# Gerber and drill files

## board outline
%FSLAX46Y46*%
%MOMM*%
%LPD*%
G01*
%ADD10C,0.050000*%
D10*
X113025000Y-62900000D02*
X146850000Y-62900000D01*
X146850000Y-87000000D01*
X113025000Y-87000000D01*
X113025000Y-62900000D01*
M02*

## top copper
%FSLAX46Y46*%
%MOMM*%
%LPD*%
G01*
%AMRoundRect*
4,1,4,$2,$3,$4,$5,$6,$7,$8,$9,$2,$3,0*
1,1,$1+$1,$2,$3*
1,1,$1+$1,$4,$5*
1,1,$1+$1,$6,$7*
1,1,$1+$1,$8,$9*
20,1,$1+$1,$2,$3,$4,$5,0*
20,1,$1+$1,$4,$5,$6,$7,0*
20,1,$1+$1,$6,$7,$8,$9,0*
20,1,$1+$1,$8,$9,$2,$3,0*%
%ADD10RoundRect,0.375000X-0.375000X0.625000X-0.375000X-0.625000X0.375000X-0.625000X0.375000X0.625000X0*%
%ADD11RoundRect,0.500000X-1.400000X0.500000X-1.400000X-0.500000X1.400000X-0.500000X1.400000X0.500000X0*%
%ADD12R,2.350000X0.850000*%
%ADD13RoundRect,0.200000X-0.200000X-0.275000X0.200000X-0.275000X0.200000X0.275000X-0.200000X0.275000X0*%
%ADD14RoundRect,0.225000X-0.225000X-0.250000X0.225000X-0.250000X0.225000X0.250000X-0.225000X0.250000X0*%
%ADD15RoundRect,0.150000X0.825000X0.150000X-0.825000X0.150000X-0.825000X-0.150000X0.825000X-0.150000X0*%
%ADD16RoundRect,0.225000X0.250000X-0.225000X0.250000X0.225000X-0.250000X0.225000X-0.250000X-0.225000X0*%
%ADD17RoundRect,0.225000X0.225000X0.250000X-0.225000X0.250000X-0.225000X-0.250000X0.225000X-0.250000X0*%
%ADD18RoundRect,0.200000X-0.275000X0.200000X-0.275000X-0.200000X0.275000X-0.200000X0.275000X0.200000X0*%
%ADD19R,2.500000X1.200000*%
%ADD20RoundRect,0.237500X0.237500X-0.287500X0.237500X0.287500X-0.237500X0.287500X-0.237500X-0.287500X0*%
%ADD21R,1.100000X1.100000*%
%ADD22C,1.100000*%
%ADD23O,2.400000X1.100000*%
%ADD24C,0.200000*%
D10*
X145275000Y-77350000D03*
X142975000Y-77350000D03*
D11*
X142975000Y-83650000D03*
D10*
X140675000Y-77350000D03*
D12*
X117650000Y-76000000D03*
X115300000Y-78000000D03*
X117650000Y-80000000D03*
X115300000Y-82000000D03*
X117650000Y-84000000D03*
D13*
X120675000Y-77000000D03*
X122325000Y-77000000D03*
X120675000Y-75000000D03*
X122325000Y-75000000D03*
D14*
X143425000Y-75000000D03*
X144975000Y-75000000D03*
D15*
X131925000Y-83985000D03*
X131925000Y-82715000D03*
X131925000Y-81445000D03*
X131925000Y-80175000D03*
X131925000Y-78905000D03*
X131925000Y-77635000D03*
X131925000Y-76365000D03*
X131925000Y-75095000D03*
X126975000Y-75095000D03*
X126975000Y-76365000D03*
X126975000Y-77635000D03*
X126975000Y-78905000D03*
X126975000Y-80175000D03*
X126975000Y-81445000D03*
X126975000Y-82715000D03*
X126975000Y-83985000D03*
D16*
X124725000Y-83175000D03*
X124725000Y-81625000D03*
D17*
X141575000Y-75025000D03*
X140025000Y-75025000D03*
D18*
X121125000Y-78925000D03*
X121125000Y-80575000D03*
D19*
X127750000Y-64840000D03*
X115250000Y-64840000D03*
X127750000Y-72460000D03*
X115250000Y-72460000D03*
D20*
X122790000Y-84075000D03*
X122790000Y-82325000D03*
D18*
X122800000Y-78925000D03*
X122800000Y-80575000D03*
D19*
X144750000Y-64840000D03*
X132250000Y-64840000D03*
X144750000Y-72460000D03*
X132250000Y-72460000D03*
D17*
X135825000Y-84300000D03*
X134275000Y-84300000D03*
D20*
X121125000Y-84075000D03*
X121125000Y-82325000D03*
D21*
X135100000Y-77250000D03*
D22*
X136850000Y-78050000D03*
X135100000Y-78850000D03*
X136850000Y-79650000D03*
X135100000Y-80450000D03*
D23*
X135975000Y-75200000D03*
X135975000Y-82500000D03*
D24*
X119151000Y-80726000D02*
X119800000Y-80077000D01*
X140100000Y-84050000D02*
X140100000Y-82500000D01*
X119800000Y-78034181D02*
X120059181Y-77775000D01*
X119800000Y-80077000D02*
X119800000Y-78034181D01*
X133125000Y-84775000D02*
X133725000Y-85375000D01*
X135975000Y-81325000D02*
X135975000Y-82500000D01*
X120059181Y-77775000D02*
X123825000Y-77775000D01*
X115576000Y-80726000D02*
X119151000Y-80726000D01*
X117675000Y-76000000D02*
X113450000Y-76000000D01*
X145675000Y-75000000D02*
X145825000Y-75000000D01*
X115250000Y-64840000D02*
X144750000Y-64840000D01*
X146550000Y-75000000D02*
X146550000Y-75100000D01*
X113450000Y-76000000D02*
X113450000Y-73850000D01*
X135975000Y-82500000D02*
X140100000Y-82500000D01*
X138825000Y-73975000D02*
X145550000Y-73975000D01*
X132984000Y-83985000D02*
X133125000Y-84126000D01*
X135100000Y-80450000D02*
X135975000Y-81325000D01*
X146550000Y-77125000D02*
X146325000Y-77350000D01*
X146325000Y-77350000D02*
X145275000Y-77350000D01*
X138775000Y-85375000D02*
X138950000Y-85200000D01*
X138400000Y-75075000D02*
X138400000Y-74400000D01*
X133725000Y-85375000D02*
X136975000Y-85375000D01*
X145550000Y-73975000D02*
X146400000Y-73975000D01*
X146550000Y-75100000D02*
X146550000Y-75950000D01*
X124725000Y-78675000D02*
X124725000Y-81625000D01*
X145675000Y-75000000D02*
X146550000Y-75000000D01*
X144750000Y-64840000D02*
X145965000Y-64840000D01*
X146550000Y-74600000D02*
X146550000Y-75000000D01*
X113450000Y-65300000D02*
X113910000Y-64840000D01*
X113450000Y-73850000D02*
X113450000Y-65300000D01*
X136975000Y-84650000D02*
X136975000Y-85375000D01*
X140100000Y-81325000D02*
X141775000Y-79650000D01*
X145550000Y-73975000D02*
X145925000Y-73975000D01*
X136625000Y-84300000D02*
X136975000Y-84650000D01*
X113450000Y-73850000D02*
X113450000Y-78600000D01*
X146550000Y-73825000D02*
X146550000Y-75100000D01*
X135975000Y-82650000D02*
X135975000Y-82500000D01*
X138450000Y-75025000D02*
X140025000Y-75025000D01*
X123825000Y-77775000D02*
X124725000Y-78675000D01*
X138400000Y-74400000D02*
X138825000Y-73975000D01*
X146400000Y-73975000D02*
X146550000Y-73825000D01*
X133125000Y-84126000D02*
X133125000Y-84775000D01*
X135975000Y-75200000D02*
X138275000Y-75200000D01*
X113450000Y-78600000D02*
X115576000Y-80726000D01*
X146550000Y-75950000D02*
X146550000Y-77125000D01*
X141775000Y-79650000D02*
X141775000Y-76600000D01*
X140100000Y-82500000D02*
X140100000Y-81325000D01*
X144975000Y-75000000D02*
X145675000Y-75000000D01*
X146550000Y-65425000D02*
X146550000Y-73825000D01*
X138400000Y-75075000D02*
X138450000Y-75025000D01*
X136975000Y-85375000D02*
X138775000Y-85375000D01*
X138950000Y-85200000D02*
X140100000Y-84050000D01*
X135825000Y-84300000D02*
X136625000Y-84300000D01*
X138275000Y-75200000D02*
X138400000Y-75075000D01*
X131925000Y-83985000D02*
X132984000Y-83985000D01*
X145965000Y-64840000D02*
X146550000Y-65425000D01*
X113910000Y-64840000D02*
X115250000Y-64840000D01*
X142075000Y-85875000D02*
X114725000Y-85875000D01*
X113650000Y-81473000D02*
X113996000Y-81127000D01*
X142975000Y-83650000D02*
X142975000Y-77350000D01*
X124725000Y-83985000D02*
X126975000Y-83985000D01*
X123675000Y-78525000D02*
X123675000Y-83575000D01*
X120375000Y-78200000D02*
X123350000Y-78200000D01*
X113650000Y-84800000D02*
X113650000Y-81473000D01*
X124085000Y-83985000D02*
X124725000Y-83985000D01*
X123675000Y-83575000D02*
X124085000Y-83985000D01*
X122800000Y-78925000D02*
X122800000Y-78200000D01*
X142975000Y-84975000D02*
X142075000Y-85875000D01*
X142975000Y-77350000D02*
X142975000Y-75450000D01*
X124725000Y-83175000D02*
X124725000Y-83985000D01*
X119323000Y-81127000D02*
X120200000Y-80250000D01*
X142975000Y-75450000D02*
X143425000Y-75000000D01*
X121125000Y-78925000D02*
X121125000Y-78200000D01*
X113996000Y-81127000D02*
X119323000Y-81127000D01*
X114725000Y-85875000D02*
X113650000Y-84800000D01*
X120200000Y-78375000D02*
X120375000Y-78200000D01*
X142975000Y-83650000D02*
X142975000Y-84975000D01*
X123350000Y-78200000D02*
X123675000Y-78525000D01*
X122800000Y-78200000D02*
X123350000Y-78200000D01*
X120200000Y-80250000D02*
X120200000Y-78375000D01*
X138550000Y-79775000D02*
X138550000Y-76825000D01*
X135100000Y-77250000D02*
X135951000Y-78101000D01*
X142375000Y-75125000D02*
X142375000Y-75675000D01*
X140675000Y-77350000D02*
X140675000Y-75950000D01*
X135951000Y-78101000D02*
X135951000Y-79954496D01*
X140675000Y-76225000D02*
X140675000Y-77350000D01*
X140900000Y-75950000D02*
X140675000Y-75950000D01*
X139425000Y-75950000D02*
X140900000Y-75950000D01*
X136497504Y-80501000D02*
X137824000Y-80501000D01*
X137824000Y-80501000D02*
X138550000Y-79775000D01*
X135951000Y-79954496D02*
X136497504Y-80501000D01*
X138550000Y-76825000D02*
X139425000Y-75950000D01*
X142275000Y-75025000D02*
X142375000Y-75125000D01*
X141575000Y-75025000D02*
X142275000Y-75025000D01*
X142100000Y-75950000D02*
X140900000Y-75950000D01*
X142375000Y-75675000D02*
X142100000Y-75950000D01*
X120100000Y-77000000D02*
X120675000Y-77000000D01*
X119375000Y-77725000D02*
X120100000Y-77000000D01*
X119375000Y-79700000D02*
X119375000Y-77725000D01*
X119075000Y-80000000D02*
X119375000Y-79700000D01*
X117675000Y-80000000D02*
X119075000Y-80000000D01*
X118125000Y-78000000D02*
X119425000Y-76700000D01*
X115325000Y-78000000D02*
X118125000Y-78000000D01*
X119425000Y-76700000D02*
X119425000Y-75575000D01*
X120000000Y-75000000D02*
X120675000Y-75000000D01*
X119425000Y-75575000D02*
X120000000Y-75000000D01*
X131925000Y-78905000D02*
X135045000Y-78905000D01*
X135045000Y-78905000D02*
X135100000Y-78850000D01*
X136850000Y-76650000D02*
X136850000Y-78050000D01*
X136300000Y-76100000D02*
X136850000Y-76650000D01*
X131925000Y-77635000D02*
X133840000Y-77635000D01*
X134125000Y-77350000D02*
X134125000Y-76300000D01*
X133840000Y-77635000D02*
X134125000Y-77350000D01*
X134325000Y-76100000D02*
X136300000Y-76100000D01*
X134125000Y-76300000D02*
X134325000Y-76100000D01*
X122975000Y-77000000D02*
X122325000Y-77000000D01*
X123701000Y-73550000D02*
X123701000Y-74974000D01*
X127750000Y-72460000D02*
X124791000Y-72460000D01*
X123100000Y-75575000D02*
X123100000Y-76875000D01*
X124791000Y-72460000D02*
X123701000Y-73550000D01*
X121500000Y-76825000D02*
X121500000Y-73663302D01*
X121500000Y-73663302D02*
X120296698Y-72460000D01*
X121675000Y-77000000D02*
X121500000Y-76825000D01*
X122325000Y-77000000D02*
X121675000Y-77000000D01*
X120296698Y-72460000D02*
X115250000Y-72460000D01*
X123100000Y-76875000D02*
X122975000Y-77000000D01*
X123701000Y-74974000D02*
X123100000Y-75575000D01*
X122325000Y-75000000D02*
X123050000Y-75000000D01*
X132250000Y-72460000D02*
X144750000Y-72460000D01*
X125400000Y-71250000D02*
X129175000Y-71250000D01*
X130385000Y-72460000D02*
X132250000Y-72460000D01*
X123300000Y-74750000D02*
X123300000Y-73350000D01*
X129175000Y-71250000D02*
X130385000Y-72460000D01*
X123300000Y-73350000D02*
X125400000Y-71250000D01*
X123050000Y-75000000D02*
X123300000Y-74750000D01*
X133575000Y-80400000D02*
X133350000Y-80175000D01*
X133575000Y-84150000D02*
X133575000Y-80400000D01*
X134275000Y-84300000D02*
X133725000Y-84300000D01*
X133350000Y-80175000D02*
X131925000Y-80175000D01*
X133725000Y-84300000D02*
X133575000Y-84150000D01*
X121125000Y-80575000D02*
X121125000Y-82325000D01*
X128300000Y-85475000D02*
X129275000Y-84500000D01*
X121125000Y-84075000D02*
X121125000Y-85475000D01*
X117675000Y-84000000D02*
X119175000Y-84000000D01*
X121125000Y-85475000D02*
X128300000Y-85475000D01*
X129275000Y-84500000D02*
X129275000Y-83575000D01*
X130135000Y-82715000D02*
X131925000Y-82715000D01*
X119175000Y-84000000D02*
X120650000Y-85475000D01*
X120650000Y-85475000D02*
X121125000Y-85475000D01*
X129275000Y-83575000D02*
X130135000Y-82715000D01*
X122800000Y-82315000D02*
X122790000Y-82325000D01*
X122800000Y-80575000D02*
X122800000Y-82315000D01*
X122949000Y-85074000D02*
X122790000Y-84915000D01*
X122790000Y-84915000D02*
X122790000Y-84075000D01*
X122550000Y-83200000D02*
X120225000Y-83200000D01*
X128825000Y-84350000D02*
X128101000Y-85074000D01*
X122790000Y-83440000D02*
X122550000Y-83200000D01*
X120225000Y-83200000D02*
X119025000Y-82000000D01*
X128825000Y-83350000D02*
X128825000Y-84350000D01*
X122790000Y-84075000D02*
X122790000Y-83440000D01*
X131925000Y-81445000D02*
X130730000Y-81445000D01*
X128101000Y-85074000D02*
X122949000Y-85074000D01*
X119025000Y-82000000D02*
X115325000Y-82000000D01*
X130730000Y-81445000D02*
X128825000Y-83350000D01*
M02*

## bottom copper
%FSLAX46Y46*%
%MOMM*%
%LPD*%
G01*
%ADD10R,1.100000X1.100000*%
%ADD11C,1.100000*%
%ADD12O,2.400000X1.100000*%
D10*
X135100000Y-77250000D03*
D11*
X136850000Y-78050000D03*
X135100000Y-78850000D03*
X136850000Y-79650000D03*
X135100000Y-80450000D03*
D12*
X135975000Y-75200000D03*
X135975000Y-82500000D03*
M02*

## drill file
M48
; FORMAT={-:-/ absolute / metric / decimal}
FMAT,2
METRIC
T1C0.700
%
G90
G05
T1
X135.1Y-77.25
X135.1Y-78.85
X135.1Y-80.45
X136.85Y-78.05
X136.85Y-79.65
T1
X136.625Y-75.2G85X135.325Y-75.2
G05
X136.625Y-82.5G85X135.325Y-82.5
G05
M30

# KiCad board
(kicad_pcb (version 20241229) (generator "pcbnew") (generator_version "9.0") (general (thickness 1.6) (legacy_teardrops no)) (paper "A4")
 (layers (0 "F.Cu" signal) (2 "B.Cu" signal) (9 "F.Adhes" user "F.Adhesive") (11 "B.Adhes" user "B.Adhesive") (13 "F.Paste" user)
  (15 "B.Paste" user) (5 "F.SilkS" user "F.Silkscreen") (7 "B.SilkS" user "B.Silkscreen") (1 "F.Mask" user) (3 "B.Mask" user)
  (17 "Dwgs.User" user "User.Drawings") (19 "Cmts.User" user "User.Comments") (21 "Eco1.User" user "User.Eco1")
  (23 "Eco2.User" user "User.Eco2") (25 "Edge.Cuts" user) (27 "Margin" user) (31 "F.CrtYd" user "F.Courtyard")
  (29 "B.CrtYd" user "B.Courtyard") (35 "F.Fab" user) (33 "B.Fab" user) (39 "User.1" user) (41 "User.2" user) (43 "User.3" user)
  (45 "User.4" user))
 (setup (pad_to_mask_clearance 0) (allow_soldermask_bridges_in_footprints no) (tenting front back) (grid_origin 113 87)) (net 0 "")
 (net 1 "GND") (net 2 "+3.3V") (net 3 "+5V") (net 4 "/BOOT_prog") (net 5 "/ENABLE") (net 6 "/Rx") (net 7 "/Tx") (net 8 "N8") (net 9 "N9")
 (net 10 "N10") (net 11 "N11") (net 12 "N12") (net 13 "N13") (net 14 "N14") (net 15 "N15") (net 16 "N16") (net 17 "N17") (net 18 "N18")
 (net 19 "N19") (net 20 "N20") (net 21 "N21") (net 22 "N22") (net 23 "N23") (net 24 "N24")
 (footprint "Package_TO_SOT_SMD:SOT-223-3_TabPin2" (layer "F.Cu") (at 142.975 80.5 -90)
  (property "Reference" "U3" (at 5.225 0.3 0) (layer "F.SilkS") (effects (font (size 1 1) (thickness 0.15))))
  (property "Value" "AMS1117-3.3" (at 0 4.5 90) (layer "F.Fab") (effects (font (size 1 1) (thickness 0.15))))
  (pad "1" smd roundrect (at -3.15 -2.3 270) (size 2 1.5) (layers "F.Cu" "F.Mask" "F.Paste") (roundrect_rratio 0.25) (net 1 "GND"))
  (pad "2" smd roundrect (at -3.15 0 270) (size 2 1.5) (layers "F.Cu" "F.Mask" "F.Paste") (roundrect_rratio 0.25) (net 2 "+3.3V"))
  (pad "2" smd roundrect (at 3.15 0 270) (size 2 3.8) (layers "F.Cu" "F.Mask" "F.Paste") (roundrect_rratio 0.25) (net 2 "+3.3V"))
  (pad "3" smd roundrect (at -3.15 2.3 270) (size 2 1.5) (layers "F.Cu" "F.Mask" "F.Paste") (roundrect_rratio 0.25) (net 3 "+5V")))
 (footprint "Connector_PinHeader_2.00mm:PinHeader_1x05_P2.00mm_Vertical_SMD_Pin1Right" (layer "F.Cu") (at 116.475 80)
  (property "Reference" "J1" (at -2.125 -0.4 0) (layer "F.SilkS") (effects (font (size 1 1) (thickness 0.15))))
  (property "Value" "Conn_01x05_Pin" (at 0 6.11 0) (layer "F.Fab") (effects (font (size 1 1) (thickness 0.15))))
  (pad "1" smd rect (at 1.175 -4) (size 2.35 0.85) (layers "F.Cu" "F.Mask" "F.Paste") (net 1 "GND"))
  (pad "2" smd rect (at -1.175 -2) (size 2.35 0.85) (layers "F.Cu" "F.Mask" "F.Paste") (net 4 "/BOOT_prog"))
  (pad "3" smd rect (at 1.175 0) (size 2.35 0.85) (layers "F.Cu" "F.Mask" "F.Paste") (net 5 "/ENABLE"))
  (pad "4" smd rect (at -1.175 2) (size 2.35 0.85) (layers "F.Cu" "F.Mask" "F.Paste") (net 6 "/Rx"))
  (pad "5" smd rect (at 1.175 4) (size 2.35 0.85) (layers "F.Cu" "F.Mask" "F.Paste") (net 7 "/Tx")))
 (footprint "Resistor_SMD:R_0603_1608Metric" (layer "F.Cu") (at 121.5 77)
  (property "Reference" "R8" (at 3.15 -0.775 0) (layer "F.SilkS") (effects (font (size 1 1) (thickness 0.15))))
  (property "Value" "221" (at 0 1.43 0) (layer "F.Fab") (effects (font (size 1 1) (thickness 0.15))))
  (pad "1" smd roundrect (at -0.825 0) (size 0.8 0.95) (layers "F.Cu" "F.Mask" "F.Paste") (roundrect_rratio 0.25) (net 5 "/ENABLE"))
  (pad "2" smd roundrect (at 0.825 0) (size 0.8 0.95) (layers "F.Cu" "F.Mask" "F.Paste") (roundrect_rratio 0.25) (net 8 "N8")))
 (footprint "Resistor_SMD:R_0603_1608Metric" (layer "F.Cu") (at 121.5 75)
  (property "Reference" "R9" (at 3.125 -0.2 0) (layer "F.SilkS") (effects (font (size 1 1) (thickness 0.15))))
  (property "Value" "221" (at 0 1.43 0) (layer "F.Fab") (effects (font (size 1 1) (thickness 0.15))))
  (pad "1" smd roundrect (at -0.825 0) (size 0.8 0.95) (layers "F.Cu" "F.Mask" "F.Paste") (roundrect_rratio 0.25) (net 4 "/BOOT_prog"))
  (pad "2" smd roundrect (at 0.825 0) (size 0.8 0.95) (layers "F.Cu" "F.Mask" "F.Paste") (roundrect_rratio 0.25) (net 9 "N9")))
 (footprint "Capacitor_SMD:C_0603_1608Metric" (layer "F.Cu") (at 144.2 75)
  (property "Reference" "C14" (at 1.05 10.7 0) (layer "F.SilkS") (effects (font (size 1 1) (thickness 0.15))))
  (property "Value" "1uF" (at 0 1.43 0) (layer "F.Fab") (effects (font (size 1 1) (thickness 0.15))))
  (pad "1" smd roundrect (at -0.775 0) (size 0.9 0.95) (layers "F.Cu" "F.Mask" "F.Paste") (roundrect_rratio 0.25) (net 2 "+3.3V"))
  (pad "2" smd roundrect (at 0.775 0) (size 0.9 0.95) (layers "F.Cu" "F.Mask" "F.Paste") (roundrect_rratio 0.25) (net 1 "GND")))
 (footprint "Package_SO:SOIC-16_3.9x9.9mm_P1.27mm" (layer "F.Cu") (at 129.45 79.54 180)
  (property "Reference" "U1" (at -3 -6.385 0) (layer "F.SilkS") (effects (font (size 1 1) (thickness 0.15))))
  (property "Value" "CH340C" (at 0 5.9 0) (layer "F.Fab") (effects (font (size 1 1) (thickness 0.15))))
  (pad "1" smd roundrect (at -2.475 -4.445 180) (size 1.95 0.6) (layers "F.Cu" "F.Mask" "F.Paste") (roundrect_rratio 0.25) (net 1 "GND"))
  (pad "2" smd roundrect (at -2.475 -3.175 180) (size 1.95 0.6) (layers "F.Cu" "F.Mask" "F.Paste") (roundrect_rratio 0.25) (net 7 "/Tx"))
  (pad "3" smd roundrect (at -2.475 -1.905 180) (size 1.95 0.6) (layers "F.Cu" "F.Mask" "F.Paste") (roundrect_rratio 0.25) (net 6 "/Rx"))
  (pad "4" smd roundrect (at -2.475 -0.635 180) (size 1.95 0.6) (layers "F.Cu" "F.Mask" "F.Paste") (roundrect_rratio 0.25) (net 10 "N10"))
  (pad "5" smd roundrect (at -2.475 0.635 180) (size 1.95 0.6) (layers "F.Cu" "F.Mask" "F.Paste") (roundrect_rratio 0.25) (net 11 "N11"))
  (pad "6" smd roundrect (at -2.475 1.905 180) (size 1.95 0.6) (layers "F.Cu" "F.Mask" "F.Paste") (roundrect_rratio 0.25) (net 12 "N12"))
  (pad "7" smd roundrect (at -2.475 3.175 180) (size 1.95 0.6) (layers "F.Cu" "F.Mask" "F.Paste") (roundrect_rratio 0.25) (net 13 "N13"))
  (pad "8" smd roundrect (at -2.475 4.445 180) (size 1.95 0.6) (layers "F.Cu" "F.Mask" "F.Paste") (roundrect_rratio 0.25) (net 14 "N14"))
  (pad "9" smd roundrect (at 2.475 4.445 180) (size 1.95 0.6) (layers "F.Cu" "F.Mask" "F.Paste") (roundrect_rratio 0.25) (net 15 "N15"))
  (pad "10" smd roundrect (at 2.475 3.175 180) (size 1.95 0.6) (layers "F.Cu" "F.Mask" "F.Paste") (roundrect_rratio 0.25) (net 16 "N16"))
  (pad "11" smd roundrect (at 2.475 1.905 180) (size 1.95 0.6) (layers "F.Cu" "F.Mask" "F.Paste") (roundrect_rratio 0.25) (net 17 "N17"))
  (pad "12" smd roundrect (at 2.475 0.635 180) (size 1.95 0.6) (layers "F.Cu" "F.Mask" "F.Paste") (roundrect_rratio 0.25) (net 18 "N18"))
  (pad "13" smd roundrect (at 2.475 -0.635 180) (size 1.95 0.6) (layers "F.Cu" "F.Mask" "F.Paste") (roundrect_rratio 0.25) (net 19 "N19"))
  (pad "14" smd roundrect (at 2.475 -1.905 180) (size 1.95 0.6) (layers "F.Cu" "F.Mask" "F.Paste") (roundrect_rratio 0.25) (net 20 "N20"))
  (pad "15" smd roundrect (at 2.475 -3.175 180) (size 1.95 0.6) (layers "F.Cu" "F.Mask" "F.Paste") (roundrect_rratio 0.25) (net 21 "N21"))
  (pad "16" smd roundrect (at 2.475 -4.445 180) (size 1.95 0.6) (layers "F.Cu" "F.Mask" "F.Paste") (roundrect_rratio 0.25) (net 2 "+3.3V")))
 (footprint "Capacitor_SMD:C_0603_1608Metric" (layer "F.Cu") (at 124.725 82.4 90)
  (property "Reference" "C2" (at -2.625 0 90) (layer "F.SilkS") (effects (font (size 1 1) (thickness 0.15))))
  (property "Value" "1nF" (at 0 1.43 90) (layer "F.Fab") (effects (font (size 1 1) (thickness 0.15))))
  (pad "1" smd roundrect (at -0.775 0 90) (size 0.9 0.95) (layers "F.Cu" "F.Mask" "F.Paste") (roundrect_rratio 0.25) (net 2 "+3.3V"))
  (pad "2" smd roundrect (at 0.775 0 90) (size 0.9 0.95) (layers "F.Cu" "F.Mask" "F.Paste") (roundrect_rratio 0.25) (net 1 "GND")))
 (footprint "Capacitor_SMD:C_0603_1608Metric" (layer "F.Cu") (at 140.8 75.025 180)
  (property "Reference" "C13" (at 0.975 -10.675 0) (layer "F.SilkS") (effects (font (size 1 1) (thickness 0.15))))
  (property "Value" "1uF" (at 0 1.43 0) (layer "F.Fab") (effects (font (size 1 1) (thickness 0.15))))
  (pad "1" smd roundrect (at -0.775 0 180) (size 0.9 0.95) (layers "F.Cu" "F.Mask" "F.Paste") (roundrect_rratio 0.25) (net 3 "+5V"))
  (pad "2" smd roundrect (at 0.775 0 180) (size 0.9 0.95) (layers "F.Cu" "F.Mask" "F.Paste") (roundrect_rratio 0.25) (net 1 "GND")))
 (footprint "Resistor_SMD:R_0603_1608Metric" (layer "F.Cu") (at 121.125 79.75 -90)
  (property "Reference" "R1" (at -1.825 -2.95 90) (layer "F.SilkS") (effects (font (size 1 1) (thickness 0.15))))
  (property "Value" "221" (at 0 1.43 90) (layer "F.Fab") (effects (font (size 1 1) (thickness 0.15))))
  (pad "1" smd roundrect (at -0.825 0 270) (size 0.8 0.95) (layers "F.Cu" "F.Mask" "F.Paste") (roundrect_rratio 0.25) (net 2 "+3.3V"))
  (pad "2" smd roundrect (at 0.825 0 270) (size 0.8 0.95) (layers "F.Cu" "F.Mask" "F.Paste") (roundrect_rratio 0.25) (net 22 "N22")))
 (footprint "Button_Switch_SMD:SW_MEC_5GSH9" (layer "F.Cu") (at 121.5 68.65 -90)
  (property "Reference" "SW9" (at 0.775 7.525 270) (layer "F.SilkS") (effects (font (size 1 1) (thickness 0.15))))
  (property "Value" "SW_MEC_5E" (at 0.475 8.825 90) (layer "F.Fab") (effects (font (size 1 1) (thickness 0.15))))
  (pad "1" smd rect (at -3.81 -6.25) (size 2.5 1.2) (layers "F.Cu" "F.Mask" "F.Paste") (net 1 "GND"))
  (pad "2" smd rect (at -3.81 6.25) (size 2.5 1.2) (layers "F.Cu" "F.Mask" "F.Paste") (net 1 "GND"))
  (pad "3" smd rect (at 3.81 -6.25) (size 2.5 1.2) (layers "F.Cu" "F.Mask" "F.Paste") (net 8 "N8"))
  (pad "4" smd rect (at 3.81 6.25) (size 2.5 1.2) (layers "F.Cu" "F.Mask" "F.Paste") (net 8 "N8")))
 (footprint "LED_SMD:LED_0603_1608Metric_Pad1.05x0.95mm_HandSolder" (layer "F.Cu") (at 122.79 83.2 90)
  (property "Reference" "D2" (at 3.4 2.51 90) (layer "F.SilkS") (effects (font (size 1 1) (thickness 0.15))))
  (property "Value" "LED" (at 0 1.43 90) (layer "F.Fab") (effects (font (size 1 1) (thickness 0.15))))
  (pad "1" smd roundrect (at -0.875 0 90) (size 1.05 0.95) (layers "F.Cu" "F.Mask" "F.Paste") (roundrect_rratio 0.25) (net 6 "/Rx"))
  (pad "2" smd roundrect (at 0.875 0 90) (size 1.05 0.95) (layers "F.Cu" "F.Mask" "F.Paste") (roundrect_rratio 0.25) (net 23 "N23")))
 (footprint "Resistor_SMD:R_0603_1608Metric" (layer "F.Cu") (at 122.8 79.75 -90)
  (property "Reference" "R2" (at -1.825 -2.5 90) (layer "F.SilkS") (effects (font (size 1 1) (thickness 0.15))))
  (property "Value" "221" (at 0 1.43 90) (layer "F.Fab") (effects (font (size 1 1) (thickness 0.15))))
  (pad "1" smd roundrect (at -0.825 0 270) (size 0.8 0.95) (layers "F.Cu" "F.Mask" "F.Paste") (roundrect_rratio 0.25) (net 2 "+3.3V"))
  (pad "2" smd roundrect (at 0.825 0 270) (size 0.8 0.95) (layers "F.Cu" "F.Mask" "F.Paste") (roundrect_rratio 0.25) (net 23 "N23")))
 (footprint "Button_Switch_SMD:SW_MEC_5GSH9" (layer "F.Cu") (at 138.5 68.65 -90)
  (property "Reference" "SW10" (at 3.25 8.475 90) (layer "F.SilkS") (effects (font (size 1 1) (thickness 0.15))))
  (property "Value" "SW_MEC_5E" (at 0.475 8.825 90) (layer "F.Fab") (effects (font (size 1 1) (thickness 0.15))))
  (pad "1" smd rect (at -3.81 -6.25) (size 2.5 1.2) (layers "F.Cu" "F.Mask" "F.Paste") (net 1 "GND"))
  (pad "2" smd rect (at -3.81 6.25) (size 2.5 1.2) (layers "F.Cu" "F.Mask" "F.Paste") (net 1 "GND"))
  (pad "3" smd rect (at 3.81 -6.25) (size 2.5 1.2) (layers "F.Cu" "F.Mask" "F.Paste") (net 9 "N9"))
  (pad "4" smd rect (at 3.81 6.25) (size 2.5 1.2) (layers "F.Cu" "F.Mask" "F.Paste") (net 9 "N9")))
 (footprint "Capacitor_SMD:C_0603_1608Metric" (layer "F.Cu") (at 135.05 84.3 180)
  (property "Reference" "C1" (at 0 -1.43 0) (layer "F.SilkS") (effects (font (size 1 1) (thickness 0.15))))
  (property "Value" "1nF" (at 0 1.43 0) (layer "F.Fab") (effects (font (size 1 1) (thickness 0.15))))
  (pad "1" smd roundrect (at -0.775 0 180) (size 0.9 0.95) (layers "F.Cu" "F.Mask" "F.Paste") (roundrect_rratio 0.25) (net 1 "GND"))
  (pad "2" smd roundrect (at 0.775 0 180) (size 0.9 0.95) (layers "F.Cu" "F.Mask" "F.Paste") (roundrect_rratio 0.25) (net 10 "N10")))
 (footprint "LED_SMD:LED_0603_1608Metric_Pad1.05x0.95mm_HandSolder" (layer "F.Cu") (at 121.125 83.2 90)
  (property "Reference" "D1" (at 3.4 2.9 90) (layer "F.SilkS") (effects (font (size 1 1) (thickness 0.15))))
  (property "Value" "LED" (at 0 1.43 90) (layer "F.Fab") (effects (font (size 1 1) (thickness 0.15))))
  (pad "1" smd roundrect (at -0.875 0 90) (size 1.05 0.95) (layers "F.Cu" "F.Mask" "F.Paste") (roundrect_rratio 0.25) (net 7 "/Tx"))
  (pad "2" smd roundrect (at 0.875 0 90) (size 1.05 0.95) (layers "F.Cu" "F.Mask" "F.Paste") (roundrect_rratio 0.25) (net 22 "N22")))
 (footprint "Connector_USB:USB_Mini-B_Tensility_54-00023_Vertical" (layer "F.Cu") (at 135.1 77.25 -90)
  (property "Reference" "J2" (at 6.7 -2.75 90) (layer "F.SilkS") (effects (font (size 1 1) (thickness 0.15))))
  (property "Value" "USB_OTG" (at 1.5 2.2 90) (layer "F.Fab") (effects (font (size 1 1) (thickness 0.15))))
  (pad "1" thru_hole rect (at 0 0 270) (size 1.1 1.1) (drill 0.7) (layers "*.Cu" "*.Mask") (remove_unused_layers no) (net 3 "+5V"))
  (pad "2" thru_hole circle (at 0.8 -1.75 270) (size 1.1 1.1) (drill 0.7) (layers "*.Cu" "*.Mask") (remove_unused_layers no) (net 12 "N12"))
  (pad "3" thru_hole circle (at 1.6 0 270) (size 1.1 1.1) (drill 0.7) (layers "*.Cu" "*.Mask") (remove_unused_layers no) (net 11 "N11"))
  (pad "4" thru_hole circle (at 2.4 -1.75 270) (size 1.1 1.1) (drill 0.7) (layers "*.Cu" "*.Mask") (remove_unused_layers no) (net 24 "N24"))
  (pad "5" thru_hole circle (at 3.2 0 270) (size 1.1 1.1) (drill 0.7) (layers "*.Cu" "*.Mask") (remove_unused_layers no) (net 1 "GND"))
  (pad "6" thru_hole oval (at -2.05 -0.875 270) (size 1.1 2.4) (drill oval 0.7 2) (layers "*.Cu" "*.Mask") (remove_unused_layers no)
   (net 1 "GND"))
  (pad "6" thru_hole oval (at 5.25 -0.875 270) (size 1.1 2.4) (drill oval 0.7 2) (layers "*.Cu" "*.Mask") (remove_unused_layers no)
   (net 1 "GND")))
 (gr_rect (start 113.025 62.9) (end 146.85 87) (stroke (width 0.05) (type default)) (fill no) (layer "Edge.Cuts"))
 (segment (start 119.151 80.726) (end 119.8 80.077) (width 0.2) (layer "F.Cu") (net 1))
 (segment (start 140.1 84.05) (end 140.1 82.5) (width 0.2) (layer "F.Cu") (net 1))
 (segment (start 119.8 78.034181) (end 120.059181 77.775) (width 0.2) (layer "F.Cu") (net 1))
 (segment (start 119.8 80.077) (end 119.8 78.034181) (width 0.2) (layer "F.Cu") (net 1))
 (segment (start 133.125 84.775) (end 133.725 85.375) (width 0.2) (layer "F.Cu") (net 1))
 (segment (start 135.975 81.325) (end 135.975 82.5) (width 0.2) (layer "F.Cu") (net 1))
 (segment (start 120.059181 77.775) (end 123.825 77.775) (width 0.2) (layer "F.Cu") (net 1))
 (segment (start 115.576 80.726) (end 119.151 80.726) (width 0.2) (layer "F.Cu") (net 1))
 (segment (start 117.675 76) (end 113.45 76) (width 0.2) (layer "F.Cu") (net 1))
 (segment (start 145.675 75) (end 145.825 75) (width 0.2) (layer "F.Cu") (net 1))
 (segment (start 115.25 64.84) (end 144.75 64.84) (width 0.2) (layer "F.Cu") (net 1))
 (segment (start 146.55 75) (end 146.55 75.1) (width 0.2) (layer "F.Cu") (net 1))
 (segment (start 113.45 76) (end 113.45 73.85) (width 0.2) (layer "F.Cu") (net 1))
 (segment (start 135.975 82.5) (end 140.1 82.5) (width 0.2) (layer "F.Cu") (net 1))
 (segment (start 138.825 73.975) (end 145.55 73.975) (width 0.2) (layer "F.Cu") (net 1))
 (segment (start 132.984 83.985) (end 133.125 84.126) (width 0.2) (layer "F.Cu") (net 1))
 (segment (start 135.1 80.45) (end 135.975 81.325) (width 0.2) (layer "F.Cu") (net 1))
 (segment (start 146.55 77.125) (end 146.325 77.35) (width 0.2) (layer "F.Cu") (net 1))
 (segment (start 146.325 77.35) (end 145.275 77.35) (width 0.2) (layer "F.Cu") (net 1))
 (segment (start 138.775 85.375) (end 138.95 85.2) (width 0.2) (layer "F.Cu") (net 1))
 (segment (start 138.4 75.075) (end 138.4 74.4) (width 0.2) (layer "F.Cu") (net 1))
 (segment (start 133.725 85.375) (end 136.975 85.375) (width 0.2) (layer "F.Cu") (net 1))
 (segment (start 145.55 73.975) (end 146.4 73.975) (width 0.2) (layer "F.Cu") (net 1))
 (segment (start 146.55 75.1) (end 146.55 75.95) (width 0.2) (layer "F.Cu") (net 1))
 (segment (start 124.725 78.675) (end 124.725 81.625) (width 0.2) (layer "F.Cu") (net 1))
 (segment (start 145.675 75) (end 146.55 75) (width 0.2) (layer "F.Cu") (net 1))
 (segment (start 144.75 64.84) (end 145.965 64.84) (width 0.2) (layer "F.Cu") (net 1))
 (segment (start 146.55 74.6) (end 146.55 75) (width 0.2) (layer "F.Cu") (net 1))
 (segment (start 113.45 65.3) (end 113.91 64.84) (width 0.2) (layer "F.Cu") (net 1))
 (segment (start 113.45 73.85) (end 113.45 65.3) (width 0.2) (layer "F.Cu") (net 1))
 (segment (start 136.975 84.65) (end 136.975 85.375) (width 0.2) (layer "F.Cu") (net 1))
 (segment (start 140.1 81.325) (end 141.775 79.65) (width 0.2) (layer "F.Cu") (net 1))
 (segment (start 145.55 73.975) (end 145.925 73.975) (width 0.2) (layer "F.Cu") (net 1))
 (segment (start 136.625 84.3) (end 136.975 84.65) (width 0.2) (layer "F.Cu") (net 1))
 (segment (start 113.45 73.85) (end 113.45 78.6) (width 0.2) (layer "F.Cu") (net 1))
 (segment (start 146.55 73.825) (end 146.55 75.1) (width 0.2) (layer "F.Cu") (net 1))
 (segment (start 135.975 82.65) (end 135.975 82.5) (width 0.2) (layer "F.Cu") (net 1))
 (segment (start 138.45 75.025) (end 140.025 75.025) (width 0.2) (layer "F.Cu") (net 1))
 (segment (start 123.825 77.775) (end 124.725 78.675) (width 0.2) (layer "F.Cu") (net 1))
 (segment (start 138.4 74.4) (end 138.825 73.975) (width 0.2) (layer "F.Cu") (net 1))
 (segment (start 146.4 73.975) (end 146.55 73.825) (width 0.2) (layer "F.Cu") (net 1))
 (segment (start 133.125 84.126) (end 133.125 84.775) (width 0.2) (layer "F.Cu") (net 1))
 (segment (start 135.975 75.2) (end 138.275 75.2) (width 0.2) (layer "F.Cu") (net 1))
 (segment (start 113.45 78.6) (end 115.576 80.726) (width 0.2) (layer "F.Cu") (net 1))
 (segment (start 146.55 75.95) (end 146.55 77.125) (width 0.2) (layer "F.Cu") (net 1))
 (segment (start 141.775 79.65) (end 141.775 76.6) (width 0.2) (layer "F.Cu") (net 1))
 (segment (start 140.1 82.5) (end 140.1 81.325) (width 0.2) (layer "F.Cu") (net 1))
 (segment (start 144.975 75) (end 145.675 75) (width 0.2) (layer "F.Cu") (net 1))
 (segment (start 146.55 65.425) (end 146.55 73.825) (width 0.2) (layer "F.Cu") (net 1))
 (segment (start 138.4 75.075) (end 138.45 75.025) (width 0.2) (layer "F.Cu") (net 1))
 (segment (start 136.975 85.375) (end 138.775 85.375) (width 0.2) (layer "F.Cu") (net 1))
 (segment (start 138.95 85.2) (end 140.1 84.05) (width 0.2) (layer "F.Cu") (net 1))
 (segment (start 135.825 84.3) (end 136.625 84.3) (width 0.2) (layer "F.Cu") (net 1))
 (segment (start 138.275 75.2) (end 138.4 75.075) (width 0.2) (layer "F.Cu") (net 1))
 (segment (start 131.925 83.985) (end 132.984 83.985) (width 0.2) (layer "F.Cu") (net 1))
 (segment (start 145.965 64.84) (end 146.55 65.425) (width 0.2) (layer "F.Cu") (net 1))
 (segment (start 113.91 64.84) (end 115.25 64.84) (width 0.2) (layer "F.Cu") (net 1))
 (segment (start 142.075 85.875) (end 114.725 85.875) (width 0.2) (layer "F.Cu") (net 2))
 (segment (start 113.65 81.473) (end 113.996 81.127) (width 0.2) (layer "F.Cu") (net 2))
 (segment (start 142.975 83.65) (end 142.975 77.35) (width 0.2) (layer "F.Cu") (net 2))
 (segment (start 124.725 83.985) (end 126.975 83.985) (width 0.2) (layer "F.Cu") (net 2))
 (segment (start 123.675 78.525) (end 123.675 83.575) (width 0.2) (layer "F.Cu") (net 2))
 (segment (start 120.375 78.2) (end 123.35 78.2) (width 0.2) (layer "F.Cu") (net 2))
 (segment (start 113.65 84.8) (end 113.65 81.473) (width 0.2) (layer "F.Cu") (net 2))
 (segment (start 124.085 83.985) (end 124.725 83.985) (width 0.2) (layer "F.Cu") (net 2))
 (segment (start 123.675 83.575) (end 124.085 83.985) (width 0.2) (layer "F.Cu") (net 2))
 (segment (start 122.8 78.925) (end 122.8 78.2) (width 0.2) (layer "F.Cu") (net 2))
 (segment (start 142.975 84.975) (end 142.075 85.875) (width 0.2) (layer "F.Cu") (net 2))
 (segment (start 142.975 77.35) (end 142.975 75.45) (width 0.2) (layer "F.Cu") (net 2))
 (segment (start 124.725 83.175) (end 124.725 83.985) (width 0.2) (layer "F.Cu") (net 2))
 (segment (start 119.323 81.127) (end 120.2 80.25) (width 0.2) (layer "F.Cu") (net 2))
 (segment (start 142.975 75.45) (end 143.425 75) (width 0.2) (layer "F.Cu") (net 2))
 (segment (start 121.125 78.925) (end 121.125 78.2) (width 0.2) (layer "F.Cu") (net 2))
 (segment (start 113.996 81.127) (end 119.323 81.127) (width 0.2) (layer "F.Cu") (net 2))
 (segment (start 114.725 85.875) (end 113.65 84.8) (width 0.2) (layer "F.Cu") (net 2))
 (segment (start 120.2 78.375) (end 120.375 78.2) (width 0.2) (layer "F.Cu") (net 2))
 (segment (start 142.975 83.65) (end 142.975 84.975) (width 0.2) (layer "F.Cu") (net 2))
 (segment (start 123.35 78.2) (end 123.675 78.525) (width 0.2) (layer "F.Cu") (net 2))
 (segment (start 122.8 78.2) (end 123.35 78.2) (width 0.2) (layer "F.Cu") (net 2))
 (segment (start 120.2 80.25) (end 120.2 78.375) (width 0.2) (layer "F.Cu") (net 2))
 (segment (start 138.55 79.775) (end 138.55 76.825) (width 0.2) (layer "F.Cu") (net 3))
 (segment (start 135.1 77.25) (end 135.951 78.101) (width 0.2) (layer "F.Cu") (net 3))
 (segment (start 142.375 75.125) (end 142.375 75.675) (width 0.2) (layer "F.Cu") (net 3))
 (segment (start 140.675 77.35) (end 140.675 75.95) (width 0.2) (layer "F.Cu") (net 3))
 (segment (start 135.951 78.101) (end 135.951 79.954496) (width 0.2) (layer "F.Cu") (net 3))
 (segment (start 140.675 76.225) (end 140.675 77.35) (width 0.2) (layer "F.Cu") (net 3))
 (segment (start 140.9 75.95) (end 140.675 75.95) (width 0.2) (layer "F.Cu") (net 3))
 (segment (start 139.425 75.95) (end 140.9 75.95) (width 0.2) (layer "F.Cu") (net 3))
 (segment (start 136.497504 80.501) (end 137.824 80.501) (width 0.2) (layer "F.Cu") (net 3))
 (segment (start 137.824 80.501) (end 138.55 79.775) (width 0.2) (layer "F.Cu") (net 3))
 (segment (start 135.951 79.954496) (end 136.497504 80.501) (width 0.2) (layer "F.Cu") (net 3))
 (segment (start 138.55 76.825) (end 139.425 75.95) (width 0.2) (layer "F.Cu") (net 3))
 (segment (start 142.275 75.025) (end 142.375 75.125) (width 0.2) (layer "F.Cu") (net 3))
 (segment (start 141.575 75.025) (end 142.275 75.025) (width 0.2) (layer "F.Cu") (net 3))
 (segment (start 142.1 75.95) (end 140.9 75.95) (width 0.2) (layer "F.Cu") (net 3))
 (segment (start 142.375 75.675) (end 142.1 75.95) (width 0.2) (layer "F.Cu") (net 3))
 (segment (start 120.1 77) (end 120.675 77) (width 0.2) (layer "F.Cu") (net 5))
 (segment (start 119.375 77.725) (end 120.1 77) (width 0.2) (layer "F.Cu") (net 5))
 (segment (start 119.375 79.7) (end 119.375 77.725) (width 0.2) (layer "F.Cu") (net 5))
 (segment (start 119.075 80) (end 119.375 79.7) (width 0.2) (layer "F.Cu") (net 5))
 (segment (start 117.675 80) (end 119.075 80) (width 0.2) (layer "F.Cu") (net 5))
 (segment (start 118.125 78) (end 119.425 76.7) (width 0.2) (layer "F.Cu") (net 4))
 (segment (start 115.325 78) (end 118.125 78) (width 0.2) (layer "F.Cu") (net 4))
 (segment (start 119.425 76.7) (end 119.425 75.575) (width 0.2) (layer "F.Cu") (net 4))
 (segment (start 120 75) (end 120.675 75) (width 0.2) (layer "F.Cu") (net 4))
 (segment (start 119.425 75.575) (end 120 75) (width 0.2) (layer "F.Cu") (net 4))
 (segment (start 131.925 78.905) (end 135.045 78.905) (width 0.2) (layer "F.Cu") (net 11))
 (segment (start 135.045 78.905) (end 135.1 78.85) (width 0.2) (layer "F.Cu") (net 11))
 (segment (start 136.85 76.65) (end 136.85 78.05) (width 0.2) (layer "F.Cu") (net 12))
 (segment (start 136.3 76.1) (end 136.85 76.65) (width 0.2) (layer "F.Cu") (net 12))
 (segment (start 131.925 77.635) (end 133.84 77.635) (width 0.2) (layer "F.Cu") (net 12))
 (segment (start 134.125 77.35) (end 134.125 76.3) (width 0.2) (layer "F.Cu") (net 12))
 (segment (start 133.84 77.635) (end 134.125 77.35) (width 0.2) (layer "F.Cu") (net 12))
 (segment (start 134.325 76.1) (end 136.3 76.1) (width 0.2) (layer "F.Cu") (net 12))
 (segment (start 134.125 76.3) (end 134.325 76.1) (width 0.2) (layer "F.Cu") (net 12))
 (segment (start 122.975 77) (end 122.325 77) (width 0.2) (layer "F.Cu") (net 8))
 (segment (start 123.701 73.55) (end 123.701 74.974) (width 0.2) (layer "F.Cu") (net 8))
 (segment (start 127.75 72.46) (end 124.791 72.46) (width 0.2) (layer "F.Cu") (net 8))
 (segment (start 123.1 75.575) (end 123.1 76.875) (width 0.2) (layer "F.Cu") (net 8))
 (segment (start 124.791 72.46) (end 123.701 73.55) (width 0.2) (layer "F.Cu") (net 8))
 (segment (start 121.5 76.825) (end 121.5 73.663302) (width 0.2) (layer "F.Cu") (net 8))
 (segment (start 121.5 73.663302) (end 120.296698 72.46) (width 0.2) (layer "F.Cu") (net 8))
 (segment (start 121.675 77) (end 121.5 76.825) (width 0.2) (layer "F.Cu") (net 8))
 (segment (start 122.325 77) (end 121.675 77) (width 0.2) (layer "F.Cu") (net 8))
 (segment (start 120.296698 72.46) (end 115.25 72.46) (width 0.2) (layer "F.Cu") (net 8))
 (segment (start 123.1 76.875) (end 122.975 77) (width 0.2) (layer "F.Cu") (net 8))
 (segment (start 123.701 74.974) (end 123.1 75.575) (width 0.2) (layer "F.Cu") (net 8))
 (segment (start 122.325 75) (end 123.05 75) (width 0.2) (layer "F.Cu") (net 9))
 (segment (start 132.25 72.46) (end 144.75 72.46) (width 0.2) (layer "F.Cu") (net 9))
 (segment (start 125.4 71.25) (end 129.175 71.25) (width 0.2) (layer "F.Cu") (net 9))
 (segment (start 130.385 72.46) (end 132.25 72.46) (width 0.2) (layer "F.Cu") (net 9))
 (segment (start 123.3 74.75) (end 123.3 73.35) (width 0.2) (layer "F.Cu") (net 9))
 (segment (start 129.175 71.25) (end 130.385 72.46) (width 0.2) (layer "F.Cu") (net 9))
 (segment (start 123.3 73.35) (end 125.4 71.25) (width 0.2) (layer "F.Cu") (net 9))
 (segment (start 123.05 75) (end 123.3 74.75) (width 0.2) (layer "F.Cu") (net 9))
 (segment (start 133.575 80.4) (end 133.35 80.175) (width 0.2) (layer "F.Cu") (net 10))
 (segment (start 133.575 84.15) (end 133.575 80.4) (width 0.2) (layer "F.Cu") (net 10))
 (segment (start 134.275 84.3) (end 133.725 84.3) (width 0.2) (layer "F.Cu") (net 10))
 (segment (start 133.35 80.175) (end 131.925 80.175) (width 0.2) (layer "F.Cu") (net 10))
 (segment (start 133.725 84.3) (end 133.575 84.15) (width 0.2) (layer "F.Cu") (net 10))
 (segment (start 121.125 80.575) (end 121.125 82.325) (width 0.2) (layer "F.Cu") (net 22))
 (segment (start 128.3 85.475) (end 129.275 84.5) (width 0.2) (layer "F.Cu") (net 7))
 (segment (start 121.125 84.075) (end 121.125 85.475) (width 0.2) (layer "F.Cu") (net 7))
 (segment (start 117.675 84) (end 119.175 84) (width 0.2) (layer "F.Cu") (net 7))
 (segment (start 121.125 85.475) (end 128.3 85.475) (width 0.2) (layer "F.Cu") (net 7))
 (segment (start 129.275 84.5) (end 129.275 83.575) (width 0.2) (layer "F.Cu") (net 7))
 (segment (start 130.135 82.715) (end 131.925 82.715) (width 0.2) (layer "F.Cu") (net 7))
 (segment (start 119.175 84) (end 120.65 85.475) (width 0.2) (layer "F.Cu") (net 7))
 (segment (start 120.65 85.475) (end 121.125 85.475) (width 0.2) (layer "F.Cu") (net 7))
 (segment (start 129.275 83.575) (end 130.135 82.715) (width 0.2) (layer "F.Cu") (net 7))
 (segment (start 122.8 82.315) (end 122.79 82.325) (width 0.2) (layer "F.Cu") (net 23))
 (segment (start 122.8 80.575) (end 122.8 82.315) (width 0.2) (layer "F.Cu") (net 23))
 (segment (start 122.949 85.074) (end 122.79 84.915) (width 0.2) (layer "F.Cu") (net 6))
 (segment (start 122.79 84.915) (end 122.79 84.075) (width 0.2) (layer "F.Cu") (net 6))
 (segment (start 122.55 83.2) (end 120.225 83.2) (width 0.2) (layer "F.Cu") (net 6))
 (segment (start 128.825 84.35) (end 128.101 85.074) (width 0.2) (layer "F.Cu") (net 6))
 (segment (start 122.79 83.44) (end 122.55 83.2) (width 0.2) (layer "F.Cu") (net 6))
 (segment (start 120.225 83.2) (end 119.025 82) (width 0.2) (layer "F.Cu") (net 6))
 (segment (start 128.825 83.35) (end 128.825 84.35) (width 0.2) (layer "F.Cu") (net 6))
 (segment (start 122.79 84.075) (end 122.79 83.44) (width 0.2) (layer "F.Cu") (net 6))
 (segment (start 131.925 81.445) (end 130.73 81.445) (width 0.2) (layer "F.Cu") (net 6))
 (segment (start 128.101 85.074) (end 122.949 85.074) (width 0.2) (layer "F.Cu") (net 6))
 (segment (start 119.025 82) (end 115.325 82) (width 0.2) (layer "F.Cu") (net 6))
 (segment (start 130.73 81.445) (end 128.825 83.35) (width 0.2) (layer "F.Cu") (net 6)))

